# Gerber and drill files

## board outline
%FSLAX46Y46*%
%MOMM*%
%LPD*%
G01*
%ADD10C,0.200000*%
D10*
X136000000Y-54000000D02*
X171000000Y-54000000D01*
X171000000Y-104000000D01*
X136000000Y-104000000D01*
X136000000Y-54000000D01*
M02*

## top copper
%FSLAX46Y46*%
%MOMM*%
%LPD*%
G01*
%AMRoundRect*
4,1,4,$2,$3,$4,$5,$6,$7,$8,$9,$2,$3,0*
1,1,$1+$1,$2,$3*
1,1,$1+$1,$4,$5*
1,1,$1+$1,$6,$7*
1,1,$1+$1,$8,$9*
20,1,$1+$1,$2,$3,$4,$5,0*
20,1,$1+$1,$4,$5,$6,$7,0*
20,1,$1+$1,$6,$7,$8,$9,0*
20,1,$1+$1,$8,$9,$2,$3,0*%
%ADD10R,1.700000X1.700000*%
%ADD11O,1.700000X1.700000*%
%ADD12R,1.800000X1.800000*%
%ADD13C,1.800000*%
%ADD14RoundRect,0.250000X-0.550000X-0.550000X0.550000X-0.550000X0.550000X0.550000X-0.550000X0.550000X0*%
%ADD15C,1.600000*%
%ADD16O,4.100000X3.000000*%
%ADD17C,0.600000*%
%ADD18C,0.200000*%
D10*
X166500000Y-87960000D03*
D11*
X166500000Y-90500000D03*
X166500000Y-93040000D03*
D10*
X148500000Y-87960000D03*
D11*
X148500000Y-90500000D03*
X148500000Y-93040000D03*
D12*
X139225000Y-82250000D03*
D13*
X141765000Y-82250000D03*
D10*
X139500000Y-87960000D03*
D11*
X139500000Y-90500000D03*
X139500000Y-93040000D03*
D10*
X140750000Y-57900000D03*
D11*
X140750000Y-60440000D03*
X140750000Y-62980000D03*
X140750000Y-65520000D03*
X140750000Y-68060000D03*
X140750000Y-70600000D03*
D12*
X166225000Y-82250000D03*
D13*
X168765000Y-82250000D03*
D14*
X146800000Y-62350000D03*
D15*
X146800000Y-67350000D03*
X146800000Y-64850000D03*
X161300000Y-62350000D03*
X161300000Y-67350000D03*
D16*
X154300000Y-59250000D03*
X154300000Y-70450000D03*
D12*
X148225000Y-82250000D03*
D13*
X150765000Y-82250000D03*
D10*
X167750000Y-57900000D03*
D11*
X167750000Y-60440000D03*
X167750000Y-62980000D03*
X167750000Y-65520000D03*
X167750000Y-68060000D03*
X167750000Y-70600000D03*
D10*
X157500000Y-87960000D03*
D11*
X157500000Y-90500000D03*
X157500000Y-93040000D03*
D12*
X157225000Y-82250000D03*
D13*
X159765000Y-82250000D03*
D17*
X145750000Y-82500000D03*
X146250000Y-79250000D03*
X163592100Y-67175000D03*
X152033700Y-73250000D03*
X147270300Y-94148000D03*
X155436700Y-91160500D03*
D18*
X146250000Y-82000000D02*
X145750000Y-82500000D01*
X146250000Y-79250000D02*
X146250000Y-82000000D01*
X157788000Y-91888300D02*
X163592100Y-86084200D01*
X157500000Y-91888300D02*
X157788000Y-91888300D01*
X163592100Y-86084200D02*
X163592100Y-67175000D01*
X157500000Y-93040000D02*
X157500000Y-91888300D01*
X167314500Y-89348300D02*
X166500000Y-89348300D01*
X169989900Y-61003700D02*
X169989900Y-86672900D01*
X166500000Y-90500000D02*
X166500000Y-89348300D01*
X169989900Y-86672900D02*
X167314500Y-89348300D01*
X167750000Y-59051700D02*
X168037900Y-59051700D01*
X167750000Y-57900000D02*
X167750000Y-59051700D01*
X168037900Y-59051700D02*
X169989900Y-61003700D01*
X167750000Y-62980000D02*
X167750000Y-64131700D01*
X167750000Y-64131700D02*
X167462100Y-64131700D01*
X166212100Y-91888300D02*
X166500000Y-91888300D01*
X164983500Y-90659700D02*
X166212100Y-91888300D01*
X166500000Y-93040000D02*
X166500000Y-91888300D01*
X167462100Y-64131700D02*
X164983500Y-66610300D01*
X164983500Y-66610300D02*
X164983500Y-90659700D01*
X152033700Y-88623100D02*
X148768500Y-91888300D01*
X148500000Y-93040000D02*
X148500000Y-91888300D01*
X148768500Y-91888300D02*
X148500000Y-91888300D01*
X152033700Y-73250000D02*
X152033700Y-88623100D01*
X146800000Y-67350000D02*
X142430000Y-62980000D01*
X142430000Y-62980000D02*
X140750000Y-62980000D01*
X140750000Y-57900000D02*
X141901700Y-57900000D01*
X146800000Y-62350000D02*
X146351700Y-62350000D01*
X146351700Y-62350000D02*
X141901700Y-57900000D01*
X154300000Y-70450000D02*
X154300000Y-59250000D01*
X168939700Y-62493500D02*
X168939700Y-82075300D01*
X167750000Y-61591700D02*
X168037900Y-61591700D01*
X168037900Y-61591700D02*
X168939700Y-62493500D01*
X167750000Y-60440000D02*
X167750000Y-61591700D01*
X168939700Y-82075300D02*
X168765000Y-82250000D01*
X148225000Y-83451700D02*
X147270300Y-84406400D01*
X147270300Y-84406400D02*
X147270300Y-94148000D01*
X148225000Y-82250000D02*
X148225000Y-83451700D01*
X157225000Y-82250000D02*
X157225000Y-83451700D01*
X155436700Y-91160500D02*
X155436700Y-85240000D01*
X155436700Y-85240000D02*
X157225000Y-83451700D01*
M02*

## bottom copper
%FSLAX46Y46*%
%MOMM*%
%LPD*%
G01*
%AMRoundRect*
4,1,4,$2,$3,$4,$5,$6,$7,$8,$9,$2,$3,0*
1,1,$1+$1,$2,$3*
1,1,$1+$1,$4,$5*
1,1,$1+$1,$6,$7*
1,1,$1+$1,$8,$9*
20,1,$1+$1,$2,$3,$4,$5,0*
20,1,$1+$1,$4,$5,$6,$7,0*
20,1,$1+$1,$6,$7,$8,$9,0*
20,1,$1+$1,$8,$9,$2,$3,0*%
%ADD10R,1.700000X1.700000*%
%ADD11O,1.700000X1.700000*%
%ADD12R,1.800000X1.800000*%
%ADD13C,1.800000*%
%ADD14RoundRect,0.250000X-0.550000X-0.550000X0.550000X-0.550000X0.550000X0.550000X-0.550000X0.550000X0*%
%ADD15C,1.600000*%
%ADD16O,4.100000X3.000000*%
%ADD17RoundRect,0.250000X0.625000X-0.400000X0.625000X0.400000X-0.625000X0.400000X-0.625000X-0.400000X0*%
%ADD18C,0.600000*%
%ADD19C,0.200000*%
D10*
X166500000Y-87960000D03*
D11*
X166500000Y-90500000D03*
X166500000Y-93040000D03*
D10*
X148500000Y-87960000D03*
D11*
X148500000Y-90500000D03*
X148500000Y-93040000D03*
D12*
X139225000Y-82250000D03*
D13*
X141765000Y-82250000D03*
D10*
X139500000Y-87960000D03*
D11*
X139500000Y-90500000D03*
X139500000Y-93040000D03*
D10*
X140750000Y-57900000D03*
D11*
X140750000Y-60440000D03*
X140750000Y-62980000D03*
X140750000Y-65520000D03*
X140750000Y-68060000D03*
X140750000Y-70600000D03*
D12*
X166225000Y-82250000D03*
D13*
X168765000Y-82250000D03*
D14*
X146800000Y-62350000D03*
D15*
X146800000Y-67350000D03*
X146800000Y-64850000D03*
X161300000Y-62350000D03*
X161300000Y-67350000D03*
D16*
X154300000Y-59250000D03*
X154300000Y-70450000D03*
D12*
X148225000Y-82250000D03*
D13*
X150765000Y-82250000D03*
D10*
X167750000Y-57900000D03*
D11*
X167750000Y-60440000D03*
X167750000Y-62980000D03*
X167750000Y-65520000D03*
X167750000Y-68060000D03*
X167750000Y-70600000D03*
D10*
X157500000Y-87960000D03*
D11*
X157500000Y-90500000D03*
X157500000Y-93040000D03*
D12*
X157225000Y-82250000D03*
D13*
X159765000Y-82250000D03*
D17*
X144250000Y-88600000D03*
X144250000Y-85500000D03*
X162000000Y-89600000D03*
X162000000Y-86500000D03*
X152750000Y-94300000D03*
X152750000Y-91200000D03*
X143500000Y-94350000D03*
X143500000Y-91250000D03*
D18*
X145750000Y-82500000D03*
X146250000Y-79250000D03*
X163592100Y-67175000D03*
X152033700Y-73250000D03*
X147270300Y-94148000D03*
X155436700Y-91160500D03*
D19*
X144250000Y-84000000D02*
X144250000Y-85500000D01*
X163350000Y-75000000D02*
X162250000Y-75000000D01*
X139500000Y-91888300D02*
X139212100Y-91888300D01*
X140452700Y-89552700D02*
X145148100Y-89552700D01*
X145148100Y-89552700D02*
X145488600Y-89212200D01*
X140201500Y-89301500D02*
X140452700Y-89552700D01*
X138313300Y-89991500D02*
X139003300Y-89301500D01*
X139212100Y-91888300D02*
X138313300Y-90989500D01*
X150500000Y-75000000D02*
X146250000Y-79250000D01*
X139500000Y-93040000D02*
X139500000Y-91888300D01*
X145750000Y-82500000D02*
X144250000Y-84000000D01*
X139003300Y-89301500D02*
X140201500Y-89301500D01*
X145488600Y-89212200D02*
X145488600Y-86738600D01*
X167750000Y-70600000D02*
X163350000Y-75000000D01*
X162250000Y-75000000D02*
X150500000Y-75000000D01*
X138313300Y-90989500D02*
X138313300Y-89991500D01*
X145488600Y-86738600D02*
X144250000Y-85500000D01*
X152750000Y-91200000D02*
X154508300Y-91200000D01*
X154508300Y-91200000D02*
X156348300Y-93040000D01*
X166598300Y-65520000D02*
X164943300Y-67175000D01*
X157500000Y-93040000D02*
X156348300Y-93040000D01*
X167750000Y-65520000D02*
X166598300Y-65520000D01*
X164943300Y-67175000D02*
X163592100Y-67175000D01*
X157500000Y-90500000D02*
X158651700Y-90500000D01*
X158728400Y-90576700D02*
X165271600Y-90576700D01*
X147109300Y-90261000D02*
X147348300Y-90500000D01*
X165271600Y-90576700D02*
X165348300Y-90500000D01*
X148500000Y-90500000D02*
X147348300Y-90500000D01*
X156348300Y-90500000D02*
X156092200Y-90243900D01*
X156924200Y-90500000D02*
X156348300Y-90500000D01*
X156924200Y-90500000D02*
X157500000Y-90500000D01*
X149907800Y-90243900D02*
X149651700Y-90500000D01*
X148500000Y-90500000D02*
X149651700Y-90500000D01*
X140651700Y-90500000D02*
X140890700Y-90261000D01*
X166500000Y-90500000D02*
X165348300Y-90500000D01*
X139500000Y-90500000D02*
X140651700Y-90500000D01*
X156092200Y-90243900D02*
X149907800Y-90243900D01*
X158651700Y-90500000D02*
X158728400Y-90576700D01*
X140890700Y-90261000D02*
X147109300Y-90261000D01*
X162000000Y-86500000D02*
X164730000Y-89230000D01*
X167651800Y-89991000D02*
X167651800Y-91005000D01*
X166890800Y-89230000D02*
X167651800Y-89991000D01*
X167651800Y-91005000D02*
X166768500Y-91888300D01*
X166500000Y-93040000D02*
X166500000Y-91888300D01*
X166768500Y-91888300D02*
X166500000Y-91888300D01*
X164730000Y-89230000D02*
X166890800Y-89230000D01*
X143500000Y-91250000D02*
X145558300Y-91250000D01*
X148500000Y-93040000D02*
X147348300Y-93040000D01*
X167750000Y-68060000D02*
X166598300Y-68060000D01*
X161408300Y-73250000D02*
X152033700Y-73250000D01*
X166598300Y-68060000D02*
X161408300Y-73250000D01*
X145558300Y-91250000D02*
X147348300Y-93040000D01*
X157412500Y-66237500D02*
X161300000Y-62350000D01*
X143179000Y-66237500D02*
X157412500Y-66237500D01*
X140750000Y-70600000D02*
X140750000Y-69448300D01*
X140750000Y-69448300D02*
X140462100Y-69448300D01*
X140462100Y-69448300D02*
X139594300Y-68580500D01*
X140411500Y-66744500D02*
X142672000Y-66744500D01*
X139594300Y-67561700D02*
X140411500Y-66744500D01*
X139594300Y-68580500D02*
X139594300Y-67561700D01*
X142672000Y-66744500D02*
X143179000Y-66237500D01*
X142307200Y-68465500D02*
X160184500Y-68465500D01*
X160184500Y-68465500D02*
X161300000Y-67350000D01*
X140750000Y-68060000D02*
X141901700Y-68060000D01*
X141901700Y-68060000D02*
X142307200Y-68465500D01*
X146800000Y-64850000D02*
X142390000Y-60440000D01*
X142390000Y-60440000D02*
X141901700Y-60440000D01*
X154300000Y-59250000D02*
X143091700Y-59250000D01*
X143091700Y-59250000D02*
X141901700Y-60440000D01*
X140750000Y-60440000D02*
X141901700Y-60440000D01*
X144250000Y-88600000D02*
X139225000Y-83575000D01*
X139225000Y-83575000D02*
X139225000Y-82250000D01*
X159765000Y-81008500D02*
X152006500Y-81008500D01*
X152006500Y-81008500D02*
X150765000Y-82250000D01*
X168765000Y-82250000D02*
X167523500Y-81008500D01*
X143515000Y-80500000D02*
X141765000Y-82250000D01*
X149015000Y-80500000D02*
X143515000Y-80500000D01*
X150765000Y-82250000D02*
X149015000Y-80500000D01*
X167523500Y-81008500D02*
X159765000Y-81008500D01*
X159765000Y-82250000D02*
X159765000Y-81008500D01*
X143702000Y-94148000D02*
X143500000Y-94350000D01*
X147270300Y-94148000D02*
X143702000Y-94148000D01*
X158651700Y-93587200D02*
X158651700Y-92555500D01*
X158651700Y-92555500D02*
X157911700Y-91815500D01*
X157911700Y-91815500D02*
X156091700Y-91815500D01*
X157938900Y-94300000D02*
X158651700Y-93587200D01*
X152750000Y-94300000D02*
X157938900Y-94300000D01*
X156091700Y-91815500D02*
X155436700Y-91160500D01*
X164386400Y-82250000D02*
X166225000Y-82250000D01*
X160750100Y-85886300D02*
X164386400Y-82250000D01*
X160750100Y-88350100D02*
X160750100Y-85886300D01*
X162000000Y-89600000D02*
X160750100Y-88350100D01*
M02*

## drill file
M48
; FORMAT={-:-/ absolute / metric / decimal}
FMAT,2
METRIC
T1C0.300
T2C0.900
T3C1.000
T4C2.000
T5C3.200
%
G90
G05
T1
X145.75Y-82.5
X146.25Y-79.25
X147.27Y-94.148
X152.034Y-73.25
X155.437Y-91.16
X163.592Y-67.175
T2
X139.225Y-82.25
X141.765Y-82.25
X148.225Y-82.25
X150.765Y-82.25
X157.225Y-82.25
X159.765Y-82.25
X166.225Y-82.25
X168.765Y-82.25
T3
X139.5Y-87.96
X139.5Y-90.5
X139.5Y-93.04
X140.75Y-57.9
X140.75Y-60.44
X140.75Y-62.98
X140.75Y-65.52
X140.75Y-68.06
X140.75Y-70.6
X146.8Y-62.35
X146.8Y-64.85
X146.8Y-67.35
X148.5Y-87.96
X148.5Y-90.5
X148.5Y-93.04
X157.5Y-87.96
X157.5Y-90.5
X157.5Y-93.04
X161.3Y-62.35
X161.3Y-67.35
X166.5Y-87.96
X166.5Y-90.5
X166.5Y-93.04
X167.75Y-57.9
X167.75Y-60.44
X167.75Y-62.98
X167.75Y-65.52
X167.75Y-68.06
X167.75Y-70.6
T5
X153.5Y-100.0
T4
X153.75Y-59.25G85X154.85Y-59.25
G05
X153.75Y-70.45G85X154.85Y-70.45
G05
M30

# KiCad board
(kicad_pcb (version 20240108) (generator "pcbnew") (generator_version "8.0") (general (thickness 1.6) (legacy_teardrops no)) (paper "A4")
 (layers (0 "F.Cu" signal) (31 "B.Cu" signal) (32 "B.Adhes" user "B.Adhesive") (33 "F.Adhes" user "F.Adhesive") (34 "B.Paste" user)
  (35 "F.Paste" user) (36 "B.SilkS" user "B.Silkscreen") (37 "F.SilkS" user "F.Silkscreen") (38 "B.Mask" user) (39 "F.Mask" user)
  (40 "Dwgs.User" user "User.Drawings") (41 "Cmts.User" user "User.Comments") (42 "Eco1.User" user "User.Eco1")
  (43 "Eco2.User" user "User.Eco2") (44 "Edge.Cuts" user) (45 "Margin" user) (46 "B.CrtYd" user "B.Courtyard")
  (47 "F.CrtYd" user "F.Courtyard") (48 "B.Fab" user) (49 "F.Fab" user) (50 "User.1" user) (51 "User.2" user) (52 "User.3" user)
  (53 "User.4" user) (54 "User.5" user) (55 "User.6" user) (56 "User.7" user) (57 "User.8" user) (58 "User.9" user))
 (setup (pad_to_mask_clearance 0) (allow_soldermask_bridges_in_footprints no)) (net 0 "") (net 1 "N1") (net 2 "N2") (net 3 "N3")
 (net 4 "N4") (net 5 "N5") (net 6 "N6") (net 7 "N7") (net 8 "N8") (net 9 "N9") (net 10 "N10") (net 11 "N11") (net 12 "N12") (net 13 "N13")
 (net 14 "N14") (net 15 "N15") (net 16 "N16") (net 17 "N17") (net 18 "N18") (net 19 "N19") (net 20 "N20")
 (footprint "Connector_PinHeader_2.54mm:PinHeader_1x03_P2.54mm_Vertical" (layer "F.Cu") (at 166.5 87.96)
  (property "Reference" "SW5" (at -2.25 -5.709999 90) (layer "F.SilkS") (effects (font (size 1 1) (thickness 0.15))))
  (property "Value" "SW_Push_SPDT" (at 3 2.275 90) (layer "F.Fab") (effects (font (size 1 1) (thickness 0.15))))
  (pad "1" thru_hole rect (at 0 0) (size 1.7 1.7) (drill 1) (layers "*.Cu" "*.Mask") (remove_unused_layers no) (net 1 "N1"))
  (pad "2" thru_hole oval (at 0 2.54) (size 1.7 1.7) (drill 1) (layers "*.Cu" "*.Mask") (remove_unused_layers no) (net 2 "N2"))
  (pad "3" thru_hole oval (at 0 5.08) (size 1.7 1.7) (drill 1) (layers "*.Cu" "*.Mask") (remove_unused_layers no) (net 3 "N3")))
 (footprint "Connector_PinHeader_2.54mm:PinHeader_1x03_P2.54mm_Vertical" (layer "F.Cu") (at 148.5 87.96)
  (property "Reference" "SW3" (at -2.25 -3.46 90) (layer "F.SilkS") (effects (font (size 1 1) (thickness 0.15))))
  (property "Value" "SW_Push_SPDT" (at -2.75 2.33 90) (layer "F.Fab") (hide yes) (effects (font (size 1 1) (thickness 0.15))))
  (pad "1" thru_hole rect (at 0 0) (size 1.7 1.7) (drill 1) (layers "*.Cu" "*.Mask") (remove_unused_layers no) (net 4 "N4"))
  (pad "2" thru_hole oval (at 0 2.54) (size 1.7 1.7) (drill 1) (layers "*.Cu" "*.Mask") (remove_unused_layers no) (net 2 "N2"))
  (pad "3" thru_hole oval (at 0 5.08) (size 1.7 1.7) (drill 1) (layers "*.Cu" "*.Mask") (remove_unused_layers no) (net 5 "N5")))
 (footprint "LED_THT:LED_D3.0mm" (layer "F.Cu") (at 139.225 82.25)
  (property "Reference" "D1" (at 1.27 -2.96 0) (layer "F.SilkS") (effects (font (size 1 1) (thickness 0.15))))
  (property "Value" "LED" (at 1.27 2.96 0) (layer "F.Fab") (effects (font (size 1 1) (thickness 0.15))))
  (pad "1" thru_hole rect (at 0 0) (size 1.8 1.8) (drill 0.9) (layers "*.Cu" "*.Mask") (remove_unused_layers no) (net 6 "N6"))
  (pad "2" thru_hole circle (at 2.54 0) (size 1.8 1.8) (drill 0.9) (layers "*.Cu" "*.Mask") (remove_unused_layers no) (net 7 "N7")))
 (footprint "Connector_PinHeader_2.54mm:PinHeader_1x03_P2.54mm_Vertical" (layer "F.Cu") (at 139.5 87.96)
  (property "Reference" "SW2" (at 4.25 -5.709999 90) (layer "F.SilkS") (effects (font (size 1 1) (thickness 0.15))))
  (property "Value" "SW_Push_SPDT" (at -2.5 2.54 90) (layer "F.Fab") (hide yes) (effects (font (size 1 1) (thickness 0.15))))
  (pad "1" thru_hole rect (at 0 0) (size 1.7 1.7) (drill 1) (layers "*.Cu" "*.Mask") (remove_unused_layers no) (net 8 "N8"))
  (pad "2" thru_hole oval (at 0 2.54) (size 1.7 1.7) (drill 1) (layers "*.Cu" "*.Mask") (remove_unused_layers no) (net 2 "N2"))
  (pad "3" thru_hole oval (at 0 5.08) (size 1.7 1.7) (drill 1) (layers "*.Cu" "*.Mask") (remove_unused_layers no) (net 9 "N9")))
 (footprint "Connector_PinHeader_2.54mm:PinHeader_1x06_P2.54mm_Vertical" (layer "F.Cu") (at 140.75 57.9)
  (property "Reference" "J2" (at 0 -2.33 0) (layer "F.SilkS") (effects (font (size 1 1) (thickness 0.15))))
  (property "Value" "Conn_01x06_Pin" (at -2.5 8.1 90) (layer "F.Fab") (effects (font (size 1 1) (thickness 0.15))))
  (pad "1" thru_hole rect (at 0 0) (size 1.7 1.7) (drill 1) (layers "*.Cu" "*.Mask") (remove_unused_layers no) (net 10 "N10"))
  (pad "2" thru_hole oval (at 0 2.54) (size 1.7 1.7) (drill 1) (layers "*.Cu" "*.Mask") (remove_unused_layers no) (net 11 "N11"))
  (pad "3" thru_hole oval (at 0 5.08) (size 1.7 1.7) (drill 1) (layers "*.Cu" "*.Mask") (remove_unused_layers no) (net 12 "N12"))
  (pad "4" thru_hole oval (at 0 7.62) (size 1.7 1.7) (drill 1) (layers "*.Cu" "*.Mask") (remove_unused_layers no) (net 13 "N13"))
  (pad "5" thru_hole oval (at 0 10.16) (size 1.7 1.7) (drill 1) (layers "*.Cu" "*.Mask") (remove_unused_layers no) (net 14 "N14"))
  (pad "6" thru_hole oval (at 0 12.7) (size 1.7 1.7) (drill 1) (layers "*.Cu" "*.Mask") (remove_unused_layers no) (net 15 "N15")))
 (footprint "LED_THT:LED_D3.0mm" (layer "F.Cu") (at 166.225 82.25)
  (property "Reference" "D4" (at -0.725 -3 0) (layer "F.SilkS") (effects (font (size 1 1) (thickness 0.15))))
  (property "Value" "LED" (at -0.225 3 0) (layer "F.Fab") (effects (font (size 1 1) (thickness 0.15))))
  (pad "1" thru_hole rect (at 0 0) (size 1.8 1.8) (drill 0.9) (layers "*.Cu" "*.Mask") (remove_unused_layers no) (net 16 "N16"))
  (pad "2" thru_hole circle (at 2.54 0) (size 1.8 1.8) (drill 0.9) (layers "*.Cu" "*.Mask") (remove_unused_layers no) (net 7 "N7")))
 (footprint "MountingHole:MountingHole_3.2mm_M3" (layer "F.Cu") (at 153.5 100)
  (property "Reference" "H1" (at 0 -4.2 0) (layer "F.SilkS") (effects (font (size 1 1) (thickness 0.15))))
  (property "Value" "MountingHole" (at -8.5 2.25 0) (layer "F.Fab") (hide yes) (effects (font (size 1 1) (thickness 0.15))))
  (pad "" np_thru_hole circle (at 0 0) (size 3.2 3.2) (drill 3.2) (layers "*.Cu" "*.Mask")))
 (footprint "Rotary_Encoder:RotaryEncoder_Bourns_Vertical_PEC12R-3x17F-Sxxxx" (layer "F.Cu") (at 146.8 62.35)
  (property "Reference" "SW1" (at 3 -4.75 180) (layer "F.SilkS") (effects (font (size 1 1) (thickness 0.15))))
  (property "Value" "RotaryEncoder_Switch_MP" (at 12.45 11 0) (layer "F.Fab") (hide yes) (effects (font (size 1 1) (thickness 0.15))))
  (pad "A" thru_hole roundrect (at 0 0) (size 1.6 1.6) (drill 1) (layers "*.Cu" "*.Mask") (remove_unused_layers no)
   (roundrect_rratio 0.15625) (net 10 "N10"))
  (pad "B" thru_hole circle (at 0 5) (size 1.6 1.6) (drill 1) (layers "*.Cu" "*.Mask") (remove_unused_layers no) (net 12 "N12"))
  (pad "C" thru_hole circle (at 0 2.5) (size 1.6 1.6) (drill 1) (layers "*.Cu" "*.Mask") (remove_unused_layers no) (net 11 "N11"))
  (pad "S1" thru_hole circle (at 14.5 0) (size 1.6 1.6) (drill 1) (layers "*.Cu" "*.Mask") (remove_unused_layers no) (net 15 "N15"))
  (pad "S2" thru_hole circle (at 14.5 5) (size 1.6 1.6) (drill 1) (layers "*.Cu" "*.Mask") (remove_unused_layers no) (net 14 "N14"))
  (pad "SH" thru_hole oval (at 7.5 -3.1) (size 4.1 3) (drill oval 3.1 2) (layers "*.Cu" "*.Mask") (remove_unused_layers no) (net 11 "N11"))
  (pad "SH" thru_hole oval (at 7.5 8.1) (size 4.1 3) (drill oval 3.1 2) (layers "*.Cu" "*.Mask") (remove_unused_layers no) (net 11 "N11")))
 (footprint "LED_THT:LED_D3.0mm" (layer "F.Cu") (at 148.225 82.25)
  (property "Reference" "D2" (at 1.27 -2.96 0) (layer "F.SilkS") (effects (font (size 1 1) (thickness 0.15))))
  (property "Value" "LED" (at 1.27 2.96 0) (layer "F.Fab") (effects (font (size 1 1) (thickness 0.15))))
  (pad "1" thru_hole rect (at 0 0) (size 1.8 1.8) (drill 0.9) (layers "*.Cu" "*.Mask") (remove_unused_layers no) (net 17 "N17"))
  (pad "2" thru_hole circle (at 2.54 0) (size 1.8 1.8) (drill 0.9) (layers "*.Cu" "*.Mask") (remove_unused_layers no) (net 7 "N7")))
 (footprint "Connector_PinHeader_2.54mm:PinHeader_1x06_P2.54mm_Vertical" (layer "F.Cu") (at 167.75 57.9)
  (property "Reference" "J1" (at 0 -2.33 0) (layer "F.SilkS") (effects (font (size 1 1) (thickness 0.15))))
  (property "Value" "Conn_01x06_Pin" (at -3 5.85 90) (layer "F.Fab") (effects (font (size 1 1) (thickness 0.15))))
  (pad "1" thru_hole rect (at 0 0) (size 1.7 1.7) (drill 1) (layers "*.Cu" "*.Mask") (remove_unused_layers no) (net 2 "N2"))
  (pad "2" thru_hole oval (at 0 2.54) (size 1.7 1.7) (drill 1) (layers "*.Cu" "*.Mask") (remove_unused_layers no) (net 7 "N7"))
  (pad "3" thru_hole oval (at 0 5.08) (size 1.7 1.7) (drill 1) (layers "*.Cu" "*.Mask") (remove_unused_layers no) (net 3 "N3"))
  (pad "4" thru_hole oval (at 0 7.62) (size 1.7 1.7) (drill 1) (layers "*.Cu" "*.Mask") (remove_unused_layers no) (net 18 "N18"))
  (pad "5" thru_hole oval (at 0 10.16) (size 1.7 1.7) (drill 1) (layers "*.Cu" "*.Mask") (remove_unused_layers no) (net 5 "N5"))
  (pad "6" thru_hole oval (at 0 12.7) (size 1.7 1.7) (drill 1) (layers "*.Cu" "*.Mask") (remove_unused_layers no) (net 9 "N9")))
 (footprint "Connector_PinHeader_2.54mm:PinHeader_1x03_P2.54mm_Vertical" (layer "F.Cu") (at 157.5 87.96)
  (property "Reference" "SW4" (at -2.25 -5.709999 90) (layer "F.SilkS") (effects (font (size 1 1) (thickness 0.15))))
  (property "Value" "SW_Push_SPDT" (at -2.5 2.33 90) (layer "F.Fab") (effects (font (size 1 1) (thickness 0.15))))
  (pad "1" thru_hole rect (at 0 0) (size 1.7 1.7) (drill 1) (layers "*.Cu" "*.Mask") (remove_unused_layers no) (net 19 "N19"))
  (pad "2" thru_hole oval (at 0 2.54) (size 1.7 1.7) (drill 1) (layers "*.Cu" "*.Mask") (remove_unused_layers no) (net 2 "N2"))
  (pad "3" thru_hole oval (at 0 5.08) (size 1.7 1.7) (drill 1) (layers "*.Cu" "*.Mask") (remove_unused_layers no) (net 18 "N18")))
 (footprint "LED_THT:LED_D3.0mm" (layer "F.Cu") (at 157.225 82.25)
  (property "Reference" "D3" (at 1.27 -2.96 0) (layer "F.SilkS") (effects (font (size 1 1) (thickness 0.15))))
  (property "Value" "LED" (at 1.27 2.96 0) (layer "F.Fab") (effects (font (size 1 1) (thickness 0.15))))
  (pad "1" thru_hole rect (at 0 0) (size 1.8 1.8) (drill 0.9) (layers "*.Cu" "*.Mask") (remove_unused_layers no) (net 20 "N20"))
  (pad "2" thru_hole circle (at 2.54 0) (size 1.8 1.8) (drill 0.9) (layers "*.Cu" "*.Mask") (remove_unused_layers no) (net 7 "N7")))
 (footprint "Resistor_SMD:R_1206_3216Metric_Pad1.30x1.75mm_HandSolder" (layer "B.Cu") (at 144.25 87.05 90)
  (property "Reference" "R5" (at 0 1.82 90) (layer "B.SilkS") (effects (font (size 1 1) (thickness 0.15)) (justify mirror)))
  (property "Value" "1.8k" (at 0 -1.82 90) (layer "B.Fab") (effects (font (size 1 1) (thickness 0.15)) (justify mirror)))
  (pad "1" smd roundrect (at -1.55 0 90) (size 1.3 1.75) (layers "B.Cu" "B.Paste" "B.Mask") (roundrect_rratio 0.192308) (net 6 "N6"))
  (pad "2" smd roundrect (at 1.55 0 90) (size 1.3 1.75) (layers "B.Cu" "B.Paste" "B.Mask") (roundrect_rratio 0.192308) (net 9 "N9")))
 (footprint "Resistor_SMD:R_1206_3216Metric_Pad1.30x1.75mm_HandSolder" (layer "B.Cu") (at 162 88.05 90)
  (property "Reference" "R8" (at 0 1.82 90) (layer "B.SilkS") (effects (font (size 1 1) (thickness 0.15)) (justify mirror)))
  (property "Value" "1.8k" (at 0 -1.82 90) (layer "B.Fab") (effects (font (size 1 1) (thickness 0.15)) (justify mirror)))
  (pad "1" smd roundrect (at -1.55 0 90) (size 1.3 1.75) (layers "B.Cu" "B.Paste" "B.Mask") (roundrect_rratio 0.192308) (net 16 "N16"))
  (pad "2" smd roundrect (at 1.55 0 90) (size 1.3 1.75) (layers "B.Cu" "B.Paste" "B.Mask") (roundrect_rratio 0.192308) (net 3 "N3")))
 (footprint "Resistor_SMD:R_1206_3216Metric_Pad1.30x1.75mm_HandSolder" (layer "B.Cu") (at 152.75 92.75 90)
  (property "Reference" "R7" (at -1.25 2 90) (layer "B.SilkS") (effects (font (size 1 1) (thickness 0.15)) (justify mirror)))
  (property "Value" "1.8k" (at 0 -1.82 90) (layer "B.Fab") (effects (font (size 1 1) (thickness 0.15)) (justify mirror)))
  (pad "1" smd roundrect (at -1.55 0 90) (size 1.3 1.75) (layers "B.Cu" "B.Paste" "B.Mask") (roundrect_rratio 0.192308) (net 20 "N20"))
  (pad "2" smd roundrect (at 1.55 0 90) (size 1.3 1.75) (layers "B.Cu" "B.Paste" "B.Mask") (roundrect_rratio 0.192308) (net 18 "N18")))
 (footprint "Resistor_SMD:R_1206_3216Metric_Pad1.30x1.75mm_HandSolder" (layer "B.Cu") (at 143.5 92.8 90)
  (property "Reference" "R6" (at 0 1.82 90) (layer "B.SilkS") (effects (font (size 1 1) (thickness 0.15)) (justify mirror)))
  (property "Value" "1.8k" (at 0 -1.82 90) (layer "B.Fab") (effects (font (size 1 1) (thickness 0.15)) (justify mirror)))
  (pad "1" smd roundrect (at -1.55 0 90) (size 1.3 1.75) (layers "B.Cu" "B.Paste" "B.Mask") (roundrect_rratio 0.192308) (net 17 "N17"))
  (pad "2" smd roundrect (at 1.55 0 90) (size 1.3 1.75) (layers "B.Cu" "B.Paste" "B.Mask") (roundrect_rratio 0.192308) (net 5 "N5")))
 (gr_rect (start 136 54) (end 171 104) (stroke (width 0.2) (type default)) (fill none) (layer "Edge.Cuts"))
 (segment (start 146.25 82) (end 145.75 82.5) (width 0.2) (layer "F.Cu") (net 9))
 (segment (start 146.25 79.25) (end 146.25 82) (width 0.2) (layer "F.Cu") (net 9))
 (via (at 145.75 82.5) (size 0.6) (drill 0.3) (layers "F.Cu" "B.Cu") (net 9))
 (via (at 146.25 79.25) (size 0.6) (drill 0.3) (layers "F.Cu" "B.Cu") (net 9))
 (segment (start 144.25 84) (end 144.25 85.5) (width 0.2) (layer "B.Cu") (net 9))
 (segment (start 163.35 75) (end 162.25 75) (width 0.2) (layer "B.Cu") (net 9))
 (segment (start 139.5 91.8883) (end 139.2121 91.8883) (width 0.2) (layer "B.Cu") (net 9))
 (segment (start 140.4527 89.5527) (end 145.1481 89.5527) (width 0.2) (layer "B.Cu") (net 9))
 (segment (start 145.1481 89.5527) (end 145.4886 89.2122) (width 0.2) (layer "B.Cu") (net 9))
 (segment (start 140.2015 89.3015) (end 140.4527 89.5527) (width 0.2) (layer "B.Cu") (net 9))
 (segment (start 138.3133 89.9915) (end 139.0033 89.3015) (width 0.2) (layer "B.Cu") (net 9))
 (segment (start 139.2121 91.8883) (end 138.3133 90.9895) (width 0.2) (layer "B.Cu") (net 9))
 (segment (start 150.5 75) (end 146.25 79.25) (width 0.2) (layer "B.Cu") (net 9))
 (segment (start 139.5 93.04) (end 139.5 91.8883) (width 0.2) (layer "B.Cu") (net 9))
 (segment (start 145.75 82.5) (end 144.25 84) (width 0.2) (layer "B.Cu") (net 9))
 (segment (start 139.0033 89.3015) (end 140.2015 89.3015) (width 0.2) (layer "B.Cu") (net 9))
 (segment (start 145.4886 89.2122) (end 145.4886 86.7386) (width 0.2) (layer "B.Cu") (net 9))
 (segment (start 167.75 70.6) (end 163.35 75) (width 0.2) (layer "B.Cu") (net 9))
 (segment (start 162.25 75) (end 150.5 75) (width 0.2) (layer "B.Cu") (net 9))
 (segment (start 138.3133 90.9895) (end 138.3133 89.9915) (width 0.2) (layer "B.Cu") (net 9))
 (segment (start 145.4886 86.7386) (end 144.25 85.5) (width 0.2) (layer "B.Cu") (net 9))
 (segment (start 157.788 91.8883) (end 163.5921 86.0842) (width 0.2) (layer "F.Cu") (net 18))
 (segment (start 157.5 91.8883) (end 157.788 91.8883) (width 0.2) (layer "F.Cu") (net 18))
 (segment (start 163.5921 86.0842) (end 163.5921 67.175) (width 0.2) (layer "F.Cu") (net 18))
 (segment (start 157.5 93.04) (end 157.5 91.8883) (width 0.2) (layer "F.Cu") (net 18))
 (via (at 163.5921 67.175) (size 0.6) (drill 0.3) (layers "F.Cu" "B.Cu") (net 18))
 (segment (start 152.75 91.2) (end 154.5083 91.2) (width 0.2) (layer "B.Cu") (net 18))
 (segment (start 154.5083 91.2) (end 156.3483 93.04) (width 0.2) (layer "B.Cu") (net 18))
 (segment (start 166.5983 65.52) (end 164.9433 67.175) (width 0.2) (layer "B.Cu") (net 18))
 (segment (start 157.5 93.04) (end 156.3483 93.04) (width 0.2) (layer "B.Cu") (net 18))
 (segment (start 167.75 65.52) (end 166.5983 65.52) (width 0.2) (layer "B.Cu") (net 18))
 (segment (start 164.9433 67.175) (end 163.5921 67.175) (width 0.2) (layer "B.Cu") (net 18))
 (segment (start 167.3145 89.3483) (end 166.5 89.3483) (width 0.2) (layer "F.Cu") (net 2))
 (segment (start 169.9899 61.0037) (end 169.9899 86.6729) (width 0.2) (layer "F.Cu") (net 2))
 (segment (start 166.5 90.5) (end 166.5 89.3483) (width 0.2) (layer "F.Cu") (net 2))
 (segment (start 169.9899 86.6729) (end 167.3145 89.3483) (width 0.2) (layer "F.Cu") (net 2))
 (segment (start 167.75 59.0517) (end 168.0379 59.0517) (width 0.2) (layer "F.Cu") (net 2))
 (segment (start 167.75 57.9) (end 167.75 59.0517) (width 0.2) (layer "F.Cu") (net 2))
 (segment (start 168.0379 59.0517) (end 169.9899 61.0037) (width 0.2) (layer "F.Cu") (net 2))
 (segment (start 157.5 90.5) (end 158.6517 90.5) (width 0.2) (layer "B.Cu") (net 2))
 (segment (start 158.7284 90.5767) (end 165.2716 90.5767) (width 0.2) (layer "B.Cu") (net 2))
 (segment (start 147.1093 90.261) (end 147.3483 90.5) (width 0.2) (layer "B.Cu") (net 2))
 (segment (start 165.2716 90.5767) (end 165.3483 90.5) (width 0.2) (layer "B.Cu") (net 2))
 (segment (start 148.5 90.5) (end 147.3483 90.5) (width 0.2) (layer "B.Cu") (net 2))
 (segment (start 156.3483 90.5) (end 156.0922 90.2439) (width 0.2) (layer "B.Cu") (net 2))
 (segment (start 156.9242 90.5) (end 156.3483 90.5) (width 0.2) (layer "B.Cu") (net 2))
 (segment (start 156.9242 90.5) (end 157.5 90.5) (width 0.2) (layer "B.Cu") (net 2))
 (segment (start 149.9078 90.2439) (end 149.6517 90.5) (width 0.2) (layer "B.Cu") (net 2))
 (segment (start 148.5 90.5) (end 149.6517 90.5) (width 0.2) (layer "B.Cu") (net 2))
 (segment (start 140.6517 90.5) (end 140.8907 90.261) (width 0.2) (layer "B.Cu") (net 2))
 (segment (start 166.5 90.5) (end 165.3483 90.5) (width 0.2) (layer "B.Cu") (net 2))
 (segment (start 139.5 90.5) (end 140.6517 90.5) (width 0.2) (layer "B.Cu") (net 2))
 (segment (start 156.0922 90.2439) (end 149.9078 90.2439) (width 0.2) (layer "B.Cu") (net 2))
 (segment (start 158.6517 90.5) (end 158.7284 90.5767) (width 0.2) (layer "B.Cu") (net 2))
 (segment (start 140.8907 90.261) (end 147.1093 90.261) (width 0.2) (layer "B.Cu") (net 2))
 (segment (start 167.75 62.98) (end 167.75 64.1317) (width 0.2) (layer "F.Cu") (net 3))
 (segment (start 167.75 64.1317) (end 167.4621 64.1317) (width 0.2) (layer "F.Cu") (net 3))
 (segment (start 166.2121 91.8883) (end 166.5 91.8883) (width 0.2) (layer "F.Cu") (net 3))
 (segment (start 164.9835 90.6597) (end 166.2121 91.8883) (width 0.2) (layer "F.Cu") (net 3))
 (segment (start 166.5 93.04) (end 166.5 91.8883) (width 0.2) (layer "F.Cu") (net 3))
 (segment (start 167.4621 64.1317) (end 164.9835 66.6103) (width 0.2) (layer "F.Cu") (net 3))
 (segment (start 164.9835 66.6103) (end 164.9835 90.6597) (width 0.2) (layer "F.Cu") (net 3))
 (segment (start 162 86.5) (end 164.73 89.23) (width 0.2) (layer "B.Cu") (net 3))
 (segment (start 167.6518 89.991) (end 167.6518 91.005) (width 0.2) (layer "B.Cu") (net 3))
 (segment (start 166.8908 89.23) (end 167.6518 89.991) (width 0.2) (layer "B.Cu") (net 3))
 (segment (start 167.6518 91.005) (end 166.7685 91.8883) (width 0.2) (layer "B.Cu") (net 3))
 (segment (start 166.5 93.04) (end 166.5 91.8883) (width 0.2) (layer "B.Cu") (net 3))
 (segment (start 166.7685 91.8883) (end 166.5 91.8883) (width 0.2) (layer "B.Cu") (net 3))
 (segment (start 164.73 89.23) (end 166.8908 89.23) (width 0.2) (layer "B.Cu") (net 3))
 (segment (start 152.0337 88.6231) (end 148.7685 91.8883) (width 0.2) (layer "F.Cu") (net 5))
 (segment (start 148.5 93.04) (end 148.5 91.8883) (width 0.2) (layer "F.Cu") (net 5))
 (segment (start 148.7685 91.8883) (end 148.5 91.8883) (width 0.2) (layer "F.Cu") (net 5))
 (segment (start 152.0337 73.25) (end 152.0337 88.6231) (width 0.2) (layer "F.Cu") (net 5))
 (via (at 152.0337 73.25) (size 0.6) (drill 0.3) (layers "F.Cu" "B.Cu") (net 5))
 (segment (start 143.5 91.25) (end 145.5583 91.25) (width 0.2) (layer "B.Cu") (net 5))
 (segment (start 148.5 93.04) (end 147.3483 93.04) (width 0.2) (layer "B.Cu") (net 5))
 (segment (start 167.75 68.06) (end 166.5983 68.06) (width 0.2) (layer "B.Cu") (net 5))
 (segment (start 161.4083 73.25) (end 152.0337 73.25) (width 0.2) (layer "B.Cu") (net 5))
 (segment (start 166.5983 68.06) (end 161.4083 73.25) (width 0.2) (layer "B.Cu") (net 5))
 (segment (start 145.5583 91.25) (end 147.3483 93.04) (width 0.2) (layer "B.Cu") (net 5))
 (segment (start 157.4125 66.2375) (end 161.3 62.35) (width 0.2) (layer "B.Cu") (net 15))
 (segment (start 143.179 66.2375) (end 157.4125 66.2375) (width 0.2) (layer "B.Cu") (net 15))
 (segment (start 140.75 70.6) (end 140.75 69.4483) (width 0.2) (layer "B.Cu") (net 15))
 (segment (start 140.75 69.4483) (end 140.4621 69.4483) (width 0.2) (layer "B.Cu") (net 15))
 (segment (start 140.4621 69.4483) (end 139.5943 68.5805) (width 0.2) (layer "B.Cu") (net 15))
 (segment (start 140.4115 66.7445) (end 142.672 66.7445) (width 0.2) (layer "B.Cu") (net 15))
 (segment (start 139.5943 67.5617) (end 140.4115 66.7445) (width 0.2) (layer "B.Cu") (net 15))
 (segment (start 139.5943 68.5805) (end 139.5943 67.5617) (width 0.2) (layer "B.Cu") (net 15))
 (segment (start 142.672 66.7445) (end 143.179 66.2375) (width 0.2) (layer "B.Cu") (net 15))
 (segment (start 146.8 67.35) (end 142.43 62.98) (width 0.2) (layer "F.Cu") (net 12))
 (segment (start 142.43 62.98) (end 140.75 62.98) (width 0.2) (layer "F.Cu") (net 12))
 (segment (start 142.3072 68.4655) (end 160.1845 68.4655) (width 0.2) (layer "B.Cu") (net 14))
 (segment (start 160.1845 68.4655) (end 161.3 67.35) (width 0.2) (layer "B.Cu") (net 14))
 (segment (start 140.75 68.06) (end 141.9017 68.06) (width 0.2) (layer "B.Cu") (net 14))
 (segment (start 141.9017 68.06) (end 142.3072 68.4655) (width 0.2) (layer "B.Cu") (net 14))
 (segment (start 140.75 57.9) (end 141.9017 57.9) (width 0.2) (layer "F.Cu") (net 10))
 (segment (start 146.8 62.35) (end 146.3517 62.35) (width 0.2) (layer "F.Cu") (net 10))
 (segment (start 146.3517 62.35) (end 141.9017 57.9) (width 0.2) (layer "F.Cu") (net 10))
 (segment (start 154.3 70.45) (end 154.3 59.25) (width 0.2) (layer "F.Cu") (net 11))
 (segment (start 146.8 64.85) (end 142.39 60.44) (width 0.2) (layer "B.Cu") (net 11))
 (segment (start 142.39 60.44) (end 141.9017 60.44) (width 0.2) (layer "B.Cu") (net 11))
 (segment (start 154.3 59.25) (end 143.0917 59.25) (width 0.2) (layer "B.Cu") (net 11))
 (segment (start 143.0917 59.25) (end 141.9017 60.44) (width 0.2) (layer "B.Cu") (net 11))
 (segment (start 140.75 60.44) (end 141.9017 60.44) (width 0.2) (layer "B.Cu") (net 11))
 (segment (start 144.25 88.6) (end 139.225 83.575) (width 0.2) (layer "B.Cu") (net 6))
 (segment (start 139.225 83.575) (end 139.225 82.25) (width 0.2) (layer "B.Cu") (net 6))
 (segment (start 168.9397 62.4935) (end 168.9397 82.0753) (width 0.2) (layer "F.Cu") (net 7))
 (segment (start 167.75 61.5917) (end 168.0379 61.5917) (width 0.2) (layer "F.Cu") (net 7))
 (segment (start 168.0379 61.5917) (end 168.9397 62.4935) (width 0.2) (layer "F.Cu") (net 7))
 (segment (start 167.75 60.44) (end 167.75 61.5917) (width 0.2) (layer "F.Cu") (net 7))
 (segment (start 168.9397 82.0753) (end 168.765 82.25) (width 0.2) (layer "F.Cu") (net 7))
 (segment (start 159.765 81.0085) (end 152.0065 81.0085) (width 0.2) (layer "B.Cu") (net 7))
 (segment (start 152.0065 81.0085) (end 150.765 82.25) (width 0.2) (layer "B.Cu") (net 7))
 (segment (start 168.765 82.25) (end 167.5235 81.0085) (width 0.2) (layer "B.Cu") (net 7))
 (segment (start 143.515 80.5) (end 141.765 82.25) (width 0.2) (layer "B.Cu") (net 7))
 (segment (start 149.015 80.5) (end 143.515 80.5) (width 0.2) (layer "B.Cu") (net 7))
 (segment (start 150.765 82.25) (end 149.015 80.5) (width 0.2) (layer "B.Cu") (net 7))
 (segment (start 167.5235 81.0085) (end 159.765 81.0085) (width 0.2) (layer "B.Cu") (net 7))
 (segment (start 159.765 82.25) (end 159.765 81.0085) (width 0.2) (layer "B.Cu") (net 7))
 (segment (start 148.225 83.4517) (end 147.2703 84.4064) (width 0.2) (layer "F.Cu") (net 17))
 (segment (start 147.2703 84.4064) (end 147.2703 94.148) (width 0.2) (layer "F.Cu") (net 17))
 (segment (start 148.225 82.25) (end 148.225 83.4517) (width 0.2) (layer "F.Cu") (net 17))
 (via (at 147.2703 94.148) (size 0.6) (drill 0.3) (layers "F.Cu" "B.Cu") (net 17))
 (segment (start 143.702 94.148) (end 143.5 94.35) (width 0.2) (layer "B.Cu") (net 17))
 (segment (start 147.2703 94.148) (end 143.702 94.148) (width 0.2) (layer "B.Cu") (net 17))
 (segment (start 157.225 82.25) (end 157.225 83.4517) (width 0.2) (layer "F.Cu") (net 20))
 (segment (start 155.4367 91.1605) (end 155.4367 85.24) (width 0.2) (layer "F.Cu") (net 20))
 (segment (start 155.4367 85.24) (end 157.225 83.4517) (width 0.2) (layer "F.Cu") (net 20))
 (via (at 155.4367 91.1605) (size 0.6) (drill 0.3) (layers "F.Cu" "B.Cu") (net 20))
 (segment (start 158.6517 93.5872) (end 158.6517 92.5555) (width 0.2) (layer "B.Cu") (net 20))
 (segment (start 158.6517 92.5555) (end 157.9117 91.8155) (width 0.2) (layer "B.Cu") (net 20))
 (segment (start 157.9117 91.8155) (end 156.0917 91.8155) (width 0.2) (layer "B.Cu") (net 20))
 (segment (start 157.9389 94.3) (end 158.6517 93.5872) (width 0.2) (layer "B.Cu") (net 20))
 (segment (start 152.75 94.3) (end 157.9389 94.3) (width 0.2) (layer "B.Cu") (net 20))
 (segment (start 156.0917 91.8155) (end 155.4367 91.1605) (width 0.2) (layer "B.Cu") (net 20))
 (segment (start 164.3864 82.25) (end 166.225 82.25) (width 0.2) (layer "B.Cu") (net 16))
 (segment (start 160.7501 85.8863) (end 164.3864 82.25) (width 0.2) (layer "B.Cu") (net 16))
 (segment (start 160.7501 88.3501) (end 160.7501 85.8863) (width 0.2) (layer "B.Cu") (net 16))
 (segment (start 162 89.6) (end 160.7501 88.3501) (width 0.2) (layer "B.Cu") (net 16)))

